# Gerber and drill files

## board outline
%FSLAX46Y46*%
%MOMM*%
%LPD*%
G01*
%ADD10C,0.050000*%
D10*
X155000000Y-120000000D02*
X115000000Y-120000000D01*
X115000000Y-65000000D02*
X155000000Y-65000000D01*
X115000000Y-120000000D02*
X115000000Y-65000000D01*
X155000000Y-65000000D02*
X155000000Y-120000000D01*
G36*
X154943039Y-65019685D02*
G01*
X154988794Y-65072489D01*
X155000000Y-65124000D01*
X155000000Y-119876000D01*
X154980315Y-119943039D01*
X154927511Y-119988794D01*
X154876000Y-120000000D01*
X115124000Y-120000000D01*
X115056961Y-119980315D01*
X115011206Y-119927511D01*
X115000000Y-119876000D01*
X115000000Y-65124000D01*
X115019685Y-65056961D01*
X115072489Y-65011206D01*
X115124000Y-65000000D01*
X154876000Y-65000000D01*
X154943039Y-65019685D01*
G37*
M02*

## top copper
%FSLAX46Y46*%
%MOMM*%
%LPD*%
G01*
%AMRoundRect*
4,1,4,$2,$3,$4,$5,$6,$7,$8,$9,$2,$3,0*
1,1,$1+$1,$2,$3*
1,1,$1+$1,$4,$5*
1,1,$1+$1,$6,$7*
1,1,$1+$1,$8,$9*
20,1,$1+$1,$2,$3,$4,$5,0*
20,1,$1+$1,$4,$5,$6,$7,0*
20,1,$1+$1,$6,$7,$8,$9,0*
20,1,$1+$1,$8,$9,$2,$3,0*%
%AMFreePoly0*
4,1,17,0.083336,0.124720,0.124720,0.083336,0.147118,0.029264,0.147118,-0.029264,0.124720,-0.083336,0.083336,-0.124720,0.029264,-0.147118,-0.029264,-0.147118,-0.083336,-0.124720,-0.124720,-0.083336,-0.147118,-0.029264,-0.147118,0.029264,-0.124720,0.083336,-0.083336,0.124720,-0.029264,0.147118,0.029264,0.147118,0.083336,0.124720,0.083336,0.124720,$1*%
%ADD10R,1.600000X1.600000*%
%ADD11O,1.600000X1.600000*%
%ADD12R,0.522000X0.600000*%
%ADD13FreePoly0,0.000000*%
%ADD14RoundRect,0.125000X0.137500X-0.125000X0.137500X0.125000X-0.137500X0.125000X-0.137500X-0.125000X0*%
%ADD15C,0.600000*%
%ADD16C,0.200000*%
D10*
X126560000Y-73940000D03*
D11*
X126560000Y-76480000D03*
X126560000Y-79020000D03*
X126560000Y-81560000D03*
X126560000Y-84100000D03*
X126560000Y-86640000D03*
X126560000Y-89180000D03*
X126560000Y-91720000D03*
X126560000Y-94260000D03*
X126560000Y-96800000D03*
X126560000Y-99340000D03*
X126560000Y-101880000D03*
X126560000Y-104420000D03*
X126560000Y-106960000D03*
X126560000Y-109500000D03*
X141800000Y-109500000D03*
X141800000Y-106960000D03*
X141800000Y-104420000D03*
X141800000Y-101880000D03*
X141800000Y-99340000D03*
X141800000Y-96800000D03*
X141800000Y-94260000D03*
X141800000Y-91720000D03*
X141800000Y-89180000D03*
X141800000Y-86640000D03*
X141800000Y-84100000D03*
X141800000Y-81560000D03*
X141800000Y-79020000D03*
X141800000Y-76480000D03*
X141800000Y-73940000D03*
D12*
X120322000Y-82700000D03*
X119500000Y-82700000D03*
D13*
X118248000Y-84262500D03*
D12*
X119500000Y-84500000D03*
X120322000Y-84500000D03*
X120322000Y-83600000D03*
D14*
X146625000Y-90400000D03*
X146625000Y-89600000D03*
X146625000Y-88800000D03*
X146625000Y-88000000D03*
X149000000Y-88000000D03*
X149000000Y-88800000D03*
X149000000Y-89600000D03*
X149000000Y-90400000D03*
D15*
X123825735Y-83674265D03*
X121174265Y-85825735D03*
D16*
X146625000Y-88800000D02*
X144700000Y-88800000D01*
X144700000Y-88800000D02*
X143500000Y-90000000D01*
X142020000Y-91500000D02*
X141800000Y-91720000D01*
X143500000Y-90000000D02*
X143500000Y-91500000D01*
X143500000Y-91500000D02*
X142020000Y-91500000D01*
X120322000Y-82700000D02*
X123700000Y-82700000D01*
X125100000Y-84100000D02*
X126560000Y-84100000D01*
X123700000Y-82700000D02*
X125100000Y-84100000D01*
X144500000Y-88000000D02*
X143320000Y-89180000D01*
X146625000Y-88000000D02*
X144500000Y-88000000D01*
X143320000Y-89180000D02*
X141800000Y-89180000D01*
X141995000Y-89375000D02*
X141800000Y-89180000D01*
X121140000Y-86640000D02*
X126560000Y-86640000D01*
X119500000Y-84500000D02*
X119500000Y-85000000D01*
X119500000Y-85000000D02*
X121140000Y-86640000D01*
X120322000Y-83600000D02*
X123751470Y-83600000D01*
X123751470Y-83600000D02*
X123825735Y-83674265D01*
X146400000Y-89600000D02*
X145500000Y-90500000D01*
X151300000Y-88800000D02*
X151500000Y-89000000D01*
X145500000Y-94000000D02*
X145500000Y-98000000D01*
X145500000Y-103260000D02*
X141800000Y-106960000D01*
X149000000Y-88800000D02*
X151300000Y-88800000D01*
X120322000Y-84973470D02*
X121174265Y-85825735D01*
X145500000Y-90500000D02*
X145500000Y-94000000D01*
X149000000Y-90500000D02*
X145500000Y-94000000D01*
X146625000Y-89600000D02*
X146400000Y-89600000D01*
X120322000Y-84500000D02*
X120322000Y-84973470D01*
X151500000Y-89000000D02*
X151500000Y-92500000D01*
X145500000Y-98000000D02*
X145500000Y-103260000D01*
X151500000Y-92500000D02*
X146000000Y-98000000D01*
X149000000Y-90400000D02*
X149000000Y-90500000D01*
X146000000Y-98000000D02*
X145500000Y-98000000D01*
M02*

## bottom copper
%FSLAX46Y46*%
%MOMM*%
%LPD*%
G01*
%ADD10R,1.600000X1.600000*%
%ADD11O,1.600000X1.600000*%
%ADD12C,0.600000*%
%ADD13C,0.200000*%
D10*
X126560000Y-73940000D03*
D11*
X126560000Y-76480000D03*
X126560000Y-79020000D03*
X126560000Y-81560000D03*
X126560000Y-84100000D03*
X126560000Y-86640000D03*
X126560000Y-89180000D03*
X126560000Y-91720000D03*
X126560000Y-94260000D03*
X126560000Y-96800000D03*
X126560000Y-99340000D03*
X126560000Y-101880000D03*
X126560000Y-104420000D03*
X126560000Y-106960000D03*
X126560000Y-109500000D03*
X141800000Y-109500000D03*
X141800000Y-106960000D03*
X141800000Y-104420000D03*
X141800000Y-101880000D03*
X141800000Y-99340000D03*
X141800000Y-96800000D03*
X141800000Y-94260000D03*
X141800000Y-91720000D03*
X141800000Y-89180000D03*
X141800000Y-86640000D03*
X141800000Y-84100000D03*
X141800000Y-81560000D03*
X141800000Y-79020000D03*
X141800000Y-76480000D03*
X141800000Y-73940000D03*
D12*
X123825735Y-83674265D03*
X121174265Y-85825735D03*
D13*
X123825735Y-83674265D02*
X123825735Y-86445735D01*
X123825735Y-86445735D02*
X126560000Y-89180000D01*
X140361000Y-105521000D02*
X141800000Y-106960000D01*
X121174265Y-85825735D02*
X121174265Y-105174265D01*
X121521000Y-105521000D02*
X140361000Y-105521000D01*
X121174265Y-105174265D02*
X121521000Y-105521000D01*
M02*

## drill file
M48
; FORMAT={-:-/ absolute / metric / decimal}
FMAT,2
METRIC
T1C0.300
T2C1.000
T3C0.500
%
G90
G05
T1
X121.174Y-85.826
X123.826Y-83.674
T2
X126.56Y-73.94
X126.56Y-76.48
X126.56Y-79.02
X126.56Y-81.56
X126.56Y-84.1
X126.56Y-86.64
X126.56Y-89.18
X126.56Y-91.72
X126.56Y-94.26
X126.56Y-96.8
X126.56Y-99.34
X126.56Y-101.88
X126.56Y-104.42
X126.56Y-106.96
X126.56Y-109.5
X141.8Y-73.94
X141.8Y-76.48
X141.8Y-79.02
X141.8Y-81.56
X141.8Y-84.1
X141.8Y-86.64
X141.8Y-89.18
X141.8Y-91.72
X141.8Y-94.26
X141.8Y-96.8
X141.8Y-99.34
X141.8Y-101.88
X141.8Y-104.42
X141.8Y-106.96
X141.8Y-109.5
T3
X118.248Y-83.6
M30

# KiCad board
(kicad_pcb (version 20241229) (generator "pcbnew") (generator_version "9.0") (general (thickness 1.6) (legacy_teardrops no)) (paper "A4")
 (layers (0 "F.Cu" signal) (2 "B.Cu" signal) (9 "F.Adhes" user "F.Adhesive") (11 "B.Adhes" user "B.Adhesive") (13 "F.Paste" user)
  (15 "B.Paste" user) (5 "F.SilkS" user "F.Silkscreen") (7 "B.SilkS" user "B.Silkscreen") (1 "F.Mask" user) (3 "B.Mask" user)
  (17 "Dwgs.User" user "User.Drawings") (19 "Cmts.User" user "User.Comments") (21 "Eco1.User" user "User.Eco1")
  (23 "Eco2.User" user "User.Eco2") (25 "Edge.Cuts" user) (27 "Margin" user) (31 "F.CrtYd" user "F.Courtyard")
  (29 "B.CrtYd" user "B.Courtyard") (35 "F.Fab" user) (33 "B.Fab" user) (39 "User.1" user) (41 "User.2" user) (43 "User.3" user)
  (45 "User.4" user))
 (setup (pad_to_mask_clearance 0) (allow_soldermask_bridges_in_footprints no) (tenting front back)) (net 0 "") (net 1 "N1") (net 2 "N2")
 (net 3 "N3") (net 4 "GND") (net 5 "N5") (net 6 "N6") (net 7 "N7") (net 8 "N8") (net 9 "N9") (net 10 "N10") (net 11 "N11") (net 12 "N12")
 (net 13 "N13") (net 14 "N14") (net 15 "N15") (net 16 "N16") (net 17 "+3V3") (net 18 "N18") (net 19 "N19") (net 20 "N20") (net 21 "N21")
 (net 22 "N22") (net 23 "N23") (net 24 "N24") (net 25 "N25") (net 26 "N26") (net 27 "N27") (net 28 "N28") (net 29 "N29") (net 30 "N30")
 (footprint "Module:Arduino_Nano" (layer "F.Cu") (at 126.56 73.94)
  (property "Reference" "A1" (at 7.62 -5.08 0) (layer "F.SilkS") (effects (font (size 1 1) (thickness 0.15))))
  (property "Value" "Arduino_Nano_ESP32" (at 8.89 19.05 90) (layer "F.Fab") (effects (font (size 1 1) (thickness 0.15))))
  (pad "1" thru_hole rect (at 0 0) (size 1.6 1.6) (drill 1) (layers "*.Cu" "*.Mask") (remove_unused_layers no) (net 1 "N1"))
  (pad "2" thru_hole oval (at 0 2.54) (size 1.6 1.6) (drill 1) (layers "*.Cu" "*.Mask") (remove_unused_layers no) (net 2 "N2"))
  (pad "3" thru_hole oval (at 0 5.08) (size 1.6 1.6) (drill 1) (layers "*.Cu" "*.Mask") (remove_unused_layers no) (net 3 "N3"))
  (pad "4" thru_hole oval (at 0 7.62) (size 1.6 1.6) (drill 1) (layers "*.Cu" "*.Mask") (remove_unused_layers no) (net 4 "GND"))
  (pad "5" thru_hole oval (at 0 10.16) (size 1.6 1.6) (drill 1) (layers "*.Cu" "*.Mask") (remove_unused_layers no) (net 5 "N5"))
  (pad "6" thru_hole oval (at 0 12.7) (size 1.6 1.6) (drill 1) (layers "*.Cu" "*.Mask") (remove_unused_layers no) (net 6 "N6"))
  (pad "7" thru_hole oval (at 0 15.24) (size 1.6 1.6) (drill 1) (layers "*.Cu" "*.Mask") (remove_unused_layers no) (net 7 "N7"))
  (pad "8" thru_hole oval (at 0 17.78) (size 1.6 1.6) (drill 1) (layers "*.Cu" "*.Mask") (remove_unused_layers no) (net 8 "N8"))
  (pad "9" thru_hole oval (at 0 20.32) (size 1.6 1.6) (drill 1) (layers "*.Cu" "*.Mask") (remove_unused_layers no) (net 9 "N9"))
  (pad "10" thru_hole oval (at 0 22.86) (size 1.6 1.6) (drill 1) (layers "*.Cu" "*.Mask") (remove_unused_layers no) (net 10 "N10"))
  (pad "11" thru_hole oval (at 0 25.4) (size 1.6 1.6) (drill 1) (layers "*.Cu" "*.Mask") (remove_unused_layers no) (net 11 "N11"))
  (pad "12" thru_hole oval (at 0 27.94) (size 1.6 1.6) (drill 1) (layers "*.Cu" "*.Mask") (remove_unused_layers no) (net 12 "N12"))
  (pad "13" thru_hole oval (at 0 30.48) (size 1.6 1.6) (drill 1) (layers "*.Cu" "*.Mask") (remove_unused_layers no) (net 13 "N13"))
  (pad "14" thru_hole oval (at 0 33.02) (size 1.6 1.6) (drill 1) (layers "*.Cu" "*.Mask") (remove_unused_layers no) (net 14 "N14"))
  (pad "15" thru_hole oval (at 0 35.56) (size 1.6 1.6) (drill 1) (layers "*.Cu" "*.Mask") (remove_unused_layers no) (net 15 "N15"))
  (pad "16" thru_hole oval (at 15.24 35.56) (size 1.6 1.6) (drill 1) (layers "*.Cu" "*.Mask") (remove_unused_layers no) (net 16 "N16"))
  (pad "17" thru_hole oval (at 15.24 33.02) (size 1.6 1.6) (drill 1) (layers "*.Cu" "*.Mask") (remove_unused_layers no) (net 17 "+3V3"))
  (pad "18" thru_hole oval (at 15.24 30.48) (size 1.6 1.6) (drill 1) (layers "*.Cu" "*.Mask") (remove_unused_layers no) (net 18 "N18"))
  (pad "19" thru_hole oval (at 15.24 27.94) (size 1.6 1.6) (drill 1) (layers "*.Cu" "*.Mask") (remove_unused_layers no) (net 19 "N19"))
  (pad "20" thru_hole oval (at 15.24 25.4) (size 1.6 1.6) (drill 1) (layers "*.Cu" "*.Mask") (remove_unused_layers no) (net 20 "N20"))
  (pad "21" thru_hole oval (at 15.24 22.86) (size 1.6 1.6) (drill 1) (layers "*.Cu" "*.Mask") (remove_unused_layers no) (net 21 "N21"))
  (pad "22" thru_hole oval (at 15.24 20.32) (size 1.6 1.6) (drill 1) (layers "*.Cu" "*.Mask") (remove_unused_layers no) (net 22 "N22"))
  (pad "23" thru_hole oval (at 15.24 17.78) (size 1.6 1.6) (drill 1) (layers "*.Cu" "*.Mask") (remove_unused_layers no) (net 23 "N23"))
  (pad "24" thru_hole oval (at 15.24 15.24) (size 1.6 1.6) (drill 1) (layers "*.Cu" "*.Mask") (remove_unused_layers no) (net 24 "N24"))
  (pad "25" thru_hole oval (at 15.24 12.7) (size 1.6 1.6) (drill 1) (layers "*.Cu" "*.Mask") (remove_unused_layers no) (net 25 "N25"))
  (pad "26" thru_hole oval (at 15.24 10.16) (size 1.6 1.6) (drill 1) (layers "*.Cu" "*.Mask") (remove_unused_layers no) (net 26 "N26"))
  (pad "27" thru_hole oval (at 15.24 7.62) (size 1.6 1.6) (drill 1) (layers "*.Cu" "*.Mask") (remove_unused_layers no) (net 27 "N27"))
  (pad "28" thru_hole oval (at 15.24 5.08) (size 1.6 1.6) (drill 1) (layers "*.Cu" "*.Mask") (remove_unused_layers no) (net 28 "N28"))
  (pad "29" thru_hole oval (at 15.24 2.54) (size 1.6 1.6) (drill 1) (layers "*.Cu" "*.Mask") (remove_unused_layers no) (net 4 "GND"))
  (pad "30" thru_hole oval (at 15.24 0) (size 1.6 1.6) (drill 1) (layers "*.Cu" "*.Mask") (remove_unused_layers no) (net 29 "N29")))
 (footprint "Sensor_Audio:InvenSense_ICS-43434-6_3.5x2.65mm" (layer "F.Cu") (at 118.958 83.6 -90)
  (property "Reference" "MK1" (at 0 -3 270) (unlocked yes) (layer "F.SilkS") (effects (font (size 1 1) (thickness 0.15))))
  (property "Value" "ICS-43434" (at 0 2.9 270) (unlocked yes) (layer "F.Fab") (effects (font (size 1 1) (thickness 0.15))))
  (pad "" np_thru_hole circle (at 0 0.71 270) (size 0.5 0.5) (drill 0.5) (layers "*.Mask"))
  (pad "1" smd rect (at -0.9 -1.364 270) (size 0.6 0.522) (layers "F.Cu" "F.Mask") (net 5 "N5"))
  (pad "2" smd rect (at -0.9 -0.542 270) (size 0.6 0.522) (layers "F.Cu" "F.Mask") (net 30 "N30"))
  (pad "3" smd custom (at 0.6625 0.71) (size 0.3 0.3) (layers "F.Cu" "F.Mask") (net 4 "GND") (options (clearance outline) (anchor circle))
   (primitives))
  (pad "4" smd rect (at 0.9 -0.542 270) (size 0.6 0.522) (layers "F.Cu" "F.Mask") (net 6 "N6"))
  (pad "5" smd rect (at 0.9 -1.364 270) (size 0.6 0.522) (layers "F.Cu" "F.Mask") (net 17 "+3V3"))
  (pad "6" smd rect (at 0 -1.364 270) (size 0.6 0.522) (layers "F.Cu" "F.Mask") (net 7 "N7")))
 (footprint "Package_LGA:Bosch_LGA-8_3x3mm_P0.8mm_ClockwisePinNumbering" (layer "F.Cu") (at 147.8125 89.2 90)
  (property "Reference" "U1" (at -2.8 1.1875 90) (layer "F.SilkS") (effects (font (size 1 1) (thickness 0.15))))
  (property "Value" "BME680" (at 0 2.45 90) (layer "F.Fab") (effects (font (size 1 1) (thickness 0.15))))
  (pad "1" smd roundrect (at -1.2 -1.1875 90) (size 0.5 0.525) (layers "F.Cu" "F.Mask" "F.Paste") (roundrect_rratio 0.25) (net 4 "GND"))
  (pad "2" smd roundrect (at -0.4 -1.1875 90) (size 0.5 0.525) (layers "F.Cu" "F.Mask" "F.Paste") (roundrect_rratio 0.25) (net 17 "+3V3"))
  (pad "3" smd roundrect (at 0.4 -1.1875 90) (size 0.5 0.525) (layers "F.Cu" "F.Mask" "F.Paste") (roundrect_rratio 0.25) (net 23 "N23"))
  (pad "4" smd roundrect (at 1.2 -1.1875 90) (size 0.5 0.525) (layers "F.Cu" "F.Mask" "F.Paste") (roundrect_rratio 0.25) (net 24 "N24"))
  (pad "5" smd roundrect (at 1.2 1.1875 90) (size 0.5 0.525) (layers "F.Cu" "F.Mask" "F.Paste") (roundrect_rratio 0.25) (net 4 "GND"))
  (pad "6" smd roundrect (at 0.4 1.1875 90) (size 0.5 0.525) (layers "F.Cu" "F.Mask" "F.Paste") (roundrect_rratio 0.25) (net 17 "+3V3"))
  (pad "7" smd roundrect (at -0.4 1.1875 90) (size 0.5 0.525) (layers "F.Cu" "F.Mask" "F.Paste") (roundrect_rratio 0.25) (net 4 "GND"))
  (pad "8" smd roundrect (at -1.2 1.1875 90) (size 0.5 0.525) (layers "F.Cu" "F.Mask" "F.Paste") (roundrect_rratio 0.25) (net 17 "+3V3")))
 (gr_line (start 155 120) (end 115 120) (stroke (width 0.05) (type default)) (layer "Edge.Cuts"))
 (gr_line (start 115 65) (end 155 65) (stroke (width 0.05) (type default)) (layer "Edge.Cuts"))
 (gr_line (start 115 120) (end 115 65) (stroke (width 0.05) (type default)) (layer "Edge.Cuts"))
 (gr_line (start 155 65) (end 155 120) (stroke (width 0.05) (type solid)) (layer "Edge.Cuts"))
 (segment (start 146.625 88.8) (end 144.7 88.8) (width 0.2) (layer "F.Cu") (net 23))
 (segment (start 144.7 88.8) (end 143.5 90) (width 0.2) (layer "F.Cu") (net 23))
 (segment (start 142.02 91.5) (end 141.8 91.72) (width 0.2) (layer "F.Cu") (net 23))
 (segment (start 143.5 90) (end 143.5 91.5) (width 0.2) (layer "F.Cu") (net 23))
 (segment (start 143.5 91.5) (end 142.02 91.5) (width 0.2) (layer "F.Cu") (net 23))
 (segment (start 120.322 82.7) (end 123.7 82.7) (width 0.2) (layer "F.Cu") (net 5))
 (segment (start 125.1 84.1) (end 126.56 84.1) (width 0.2) (layer "F.Cu") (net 5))
 (segment (start 123.7 82.7) (end 125.1 84.1) (width 0.2) (layer "F.Cu") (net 5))
 (segment (start 144.5 88) (end 143.32 89.18) (width 0.2) (layer "F.Cu") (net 24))
 (segment (start 146.625 88) (end 144.5 88) (width 0.2) (layer "F.Cu") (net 24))
 (segment (start 143.32 89.18) (end 141.8 89.18) (width 0.2) (layer "F.Cu") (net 24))
 (segment (start 141.995 89.375) (end 141.8 89.18) (width 0.2) (layer "F.Cu") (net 24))
 (segment (start 121.14 86.64) (end 126.56 86.64) (width 0.2) (layer "F.Cu") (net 6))
 (segment (start 119.5 84.5) (end 119.5 85) (width 0.2) (layer "F.Cu") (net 6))
 (segment (start 119.5 85) (end 121.14 86.64) (width 0.2) (layer "F.Cu") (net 6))
 (segment (start 120.322 83.6) (end 123.75147 83.6) (width 0.2) (layer "F.Cu") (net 7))
 (segment (start 123.75147 83.6) (end 123.825735 83.674265) (width 0.2) (layer "F.Cu") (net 7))
 (via (at 123.825735 83.674265) (size 0.6) (drill 0.3) (layers "F.Cu" "B.Cu") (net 7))
 (segment (start 123.825735 83.674265) (end 123.825735 86.445735) (width 0.2) (layer "B.Cu") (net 7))
 (segment (start 123.825735 86.445735) (end 126.56 89.18) (width 0.2) (layer "B.Cu") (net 7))
 (segment (start 146.4 89.6) (end 145.5 90.5) (width 0.2) (layer "F.Cu") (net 17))
 (segment (start 151.3 88.8) (end 151.5 89) (width 0.2) (layer "F.Cu") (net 17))
 (segment (start 145.5 94) (end 145.5 98) (width 0.2) (layer "F.Cu") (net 17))
 (segment (start 145.5 103.26) (end 141.8 106.96) (width 0.2) (layer "F.Cu") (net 17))
 (segment (start 149 88.8) (end 151.3 88.8) (width 0.2) (layer "F.Cu") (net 17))
 (segment (start 120.322 84.97347) (end 121.174265 85.825735) (width 0.2) (layer "F.Cu") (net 17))
 (segment (start 145.5 90.5) (end 145.5 94) (width 0.2) (layer "F.Cu") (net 17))
 (segment (start 149 90.5) (end 145.5 94) (width 0.2) (layer "F.Cu") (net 17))
 (segment (start 146.625 89.6) (end 146.4 89.6) (width 0.2) (layer "F.Cu") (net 17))
 (segment (start 120.322 84.5) (end 120.322 84.97347) (width 0.2) (layer "F.Cu") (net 17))
 (segment (start 151.5 89) (end 151.5 92.5) (width 0.2) (layer "F.Cu") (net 17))
 (segment (start 145.5 98) (end 145.5 103.26) (width 0.2) (layer "F.Cu") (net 17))
 (segment (start 151.5 92.5) (end 146 98) (width 0.2) (layer "F.Cu") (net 17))
 (segment (start 149 90.4) (end 149 90.5) (width 0.2) (layer "F.Cu") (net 17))
 (segment (start 146 98) (end 145.5 98) (width 0.2) (layer "F.Cu") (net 17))
 (via (at 121.174265 85.825735) (size 0.6) (drill 0.3) (layers "F.Cu" "B.Cu") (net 17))
 (segment (start 140.361 105.521) (end 141.8 106.96) (width 0.2) (layer "B.Cu") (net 17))
 (segment (start 121.174265 85.825735) (end 121.174265 105.174265) (width 0.2) (layer "B.Cu") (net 17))
 (segment (start 121.521 105.521) (end 140.361 105.521) (width 0.2) (layer "B.Cu") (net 17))
 (segment (start 121.174265 105.174265) (end 121.521 105.521) (width 0.2) (layer "B.Cu") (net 17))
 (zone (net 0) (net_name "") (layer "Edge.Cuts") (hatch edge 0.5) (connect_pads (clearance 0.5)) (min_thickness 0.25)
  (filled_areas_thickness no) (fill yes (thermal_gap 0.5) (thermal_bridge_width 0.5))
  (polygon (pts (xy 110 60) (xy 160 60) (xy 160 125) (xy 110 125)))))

